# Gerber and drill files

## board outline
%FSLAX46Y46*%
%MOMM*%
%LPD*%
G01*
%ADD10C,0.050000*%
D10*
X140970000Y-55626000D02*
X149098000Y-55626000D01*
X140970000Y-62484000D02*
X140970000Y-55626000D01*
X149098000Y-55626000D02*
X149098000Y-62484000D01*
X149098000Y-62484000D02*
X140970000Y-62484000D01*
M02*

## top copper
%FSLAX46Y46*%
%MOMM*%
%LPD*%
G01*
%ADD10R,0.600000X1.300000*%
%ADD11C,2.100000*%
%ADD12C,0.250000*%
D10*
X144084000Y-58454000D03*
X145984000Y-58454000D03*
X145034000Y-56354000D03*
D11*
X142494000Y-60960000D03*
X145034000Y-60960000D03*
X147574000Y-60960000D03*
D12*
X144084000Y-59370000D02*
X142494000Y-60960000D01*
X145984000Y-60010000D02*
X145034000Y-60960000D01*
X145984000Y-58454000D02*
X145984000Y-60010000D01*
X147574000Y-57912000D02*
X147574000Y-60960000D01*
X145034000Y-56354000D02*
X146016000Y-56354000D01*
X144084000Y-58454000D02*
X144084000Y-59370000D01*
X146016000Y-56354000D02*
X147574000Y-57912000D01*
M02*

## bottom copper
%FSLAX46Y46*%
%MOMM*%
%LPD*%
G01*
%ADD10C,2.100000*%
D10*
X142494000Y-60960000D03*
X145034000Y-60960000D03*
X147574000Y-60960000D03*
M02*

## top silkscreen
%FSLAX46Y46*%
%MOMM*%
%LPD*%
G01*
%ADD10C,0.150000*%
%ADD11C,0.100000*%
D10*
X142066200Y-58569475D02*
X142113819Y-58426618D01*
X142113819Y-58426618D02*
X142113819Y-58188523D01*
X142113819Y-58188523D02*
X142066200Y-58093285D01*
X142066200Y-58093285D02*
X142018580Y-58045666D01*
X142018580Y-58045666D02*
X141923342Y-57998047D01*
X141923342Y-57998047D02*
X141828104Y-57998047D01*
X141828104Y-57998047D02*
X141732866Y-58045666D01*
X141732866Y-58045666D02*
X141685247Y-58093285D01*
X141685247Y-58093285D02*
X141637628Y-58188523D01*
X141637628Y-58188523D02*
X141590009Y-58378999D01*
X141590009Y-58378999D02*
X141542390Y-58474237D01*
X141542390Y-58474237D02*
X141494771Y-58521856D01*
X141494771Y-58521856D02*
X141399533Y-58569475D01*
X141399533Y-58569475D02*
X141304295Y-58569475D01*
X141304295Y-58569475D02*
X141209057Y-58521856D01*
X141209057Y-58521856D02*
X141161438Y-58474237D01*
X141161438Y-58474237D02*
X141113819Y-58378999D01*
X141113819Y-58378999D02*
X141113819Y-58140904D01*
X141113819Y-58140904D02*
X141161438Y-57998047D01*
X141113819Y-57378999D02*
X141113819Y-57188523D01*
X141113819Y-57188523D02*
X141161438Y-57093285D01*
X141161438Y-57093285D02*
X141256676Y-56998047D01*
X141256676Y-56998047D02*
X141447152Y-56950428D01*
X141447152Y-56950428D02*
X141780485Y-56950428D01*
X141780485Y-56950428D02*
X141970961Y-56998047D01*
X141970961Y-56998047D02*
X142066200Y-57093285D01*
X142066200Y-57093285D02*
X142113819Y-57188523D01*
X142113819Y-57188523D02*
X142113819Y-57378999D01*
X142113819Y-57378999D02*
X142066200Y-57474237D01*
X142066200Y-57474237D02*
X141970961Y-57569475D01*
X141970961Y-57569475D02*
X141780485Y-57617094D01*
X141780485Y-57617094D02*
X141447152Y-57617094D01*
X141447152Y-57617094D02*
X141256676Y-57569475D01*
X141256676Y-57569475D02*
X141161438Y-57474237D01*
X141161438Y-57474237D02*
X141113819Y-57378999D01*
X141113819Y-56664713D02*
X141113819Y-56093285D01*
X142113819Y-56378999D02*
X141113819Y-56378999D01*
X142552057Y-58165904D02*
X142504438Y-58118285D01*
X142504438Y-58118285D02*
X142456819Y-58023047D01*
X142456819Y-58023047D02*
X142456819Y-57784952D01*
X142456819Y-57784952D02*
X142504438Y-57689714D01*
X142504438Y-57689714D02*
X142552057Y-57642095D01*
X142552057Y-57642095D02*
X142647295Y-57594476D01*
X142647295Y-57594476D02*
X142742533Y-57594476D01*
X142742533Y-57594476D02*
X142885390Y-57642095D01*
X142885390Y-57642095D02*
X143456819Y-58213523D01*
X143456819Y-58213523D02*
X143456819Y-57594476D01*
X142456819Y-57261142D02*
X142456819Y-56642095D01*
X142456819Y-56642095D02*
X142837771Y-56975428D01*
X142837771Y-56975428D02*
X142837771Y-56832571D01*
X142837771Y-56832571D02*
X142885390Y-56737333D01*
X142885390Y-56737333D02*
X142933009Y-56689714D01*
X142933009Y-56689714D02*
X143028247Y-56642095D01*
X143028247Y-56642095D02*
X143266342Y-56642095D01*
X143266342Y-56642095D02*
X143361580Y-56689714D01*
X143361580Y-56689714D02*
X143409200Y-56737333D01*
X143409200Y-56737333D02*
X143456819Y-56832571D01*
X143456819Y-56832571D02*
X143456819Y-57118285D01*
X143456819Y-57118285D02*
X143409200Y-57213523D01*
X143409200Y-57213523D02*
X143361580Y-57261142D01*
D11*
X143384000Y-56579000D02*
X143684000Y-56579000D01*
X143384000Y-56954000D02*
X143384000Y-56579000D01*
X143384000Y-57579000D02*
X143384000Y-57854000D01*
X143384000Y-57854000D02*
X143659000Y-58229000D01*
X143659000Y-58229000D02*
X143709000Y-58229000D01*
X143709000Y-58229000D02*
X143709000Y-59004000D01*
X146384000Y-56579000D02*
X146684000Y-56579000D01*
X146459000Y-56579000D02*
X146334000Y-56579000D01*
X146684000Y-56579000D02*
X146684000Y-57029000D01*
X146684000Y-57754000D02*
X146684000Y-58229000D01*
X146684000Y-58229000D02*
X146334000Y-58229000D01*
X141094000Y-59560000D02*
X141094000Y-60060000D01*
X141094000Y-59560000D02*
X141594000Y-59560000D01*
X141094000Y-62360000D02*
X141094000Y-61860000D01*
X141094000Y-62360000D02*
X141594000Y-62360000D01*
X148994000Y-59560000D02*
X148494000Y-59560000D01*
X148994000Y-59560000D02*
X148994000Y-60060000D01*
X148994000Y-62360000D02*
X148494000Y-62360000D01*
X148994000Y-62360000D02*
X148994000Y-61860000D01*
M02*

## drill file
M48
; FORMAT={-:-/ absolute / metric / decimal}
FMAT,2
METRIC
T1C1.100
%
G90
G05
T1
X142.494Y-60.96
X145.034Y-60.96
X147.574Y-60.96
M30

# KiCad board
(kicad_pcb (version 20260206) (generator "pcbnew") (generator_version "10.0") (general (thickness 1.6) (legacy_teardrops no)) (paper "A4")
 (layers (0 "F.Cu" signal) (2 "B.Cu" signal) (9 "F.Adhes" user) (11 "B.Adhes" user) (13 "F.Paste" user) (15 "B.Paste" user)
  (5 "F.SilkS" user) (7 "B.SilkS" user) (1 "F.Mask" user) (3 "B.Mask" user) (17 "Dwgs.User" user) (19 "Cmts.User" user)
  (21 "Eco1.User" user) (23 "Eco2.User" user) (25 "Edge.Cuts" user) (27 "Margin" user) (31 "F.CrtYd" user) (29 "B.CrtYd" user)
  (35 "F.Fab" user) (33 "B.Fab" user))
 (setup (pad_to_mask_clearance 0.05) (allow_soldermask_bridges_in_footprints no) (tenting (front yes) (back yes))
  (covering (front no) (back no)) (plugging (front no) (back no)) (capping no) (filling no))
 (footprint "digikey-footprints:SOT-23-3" (layer "F.Cu") (at 145.034 57.404 90)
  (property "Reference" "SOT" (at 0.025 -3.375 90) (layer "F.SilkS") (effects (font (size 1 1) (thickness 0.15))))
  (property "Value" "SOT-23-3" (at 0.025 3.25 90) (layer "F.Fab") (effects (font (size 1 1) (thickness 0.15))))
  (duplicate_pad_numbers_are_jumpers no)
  (fp_line (start 0.825 -1.65) (end 0.825 -1.35) (stroke (width 0.1) (type solid)) (layer "F.SilkS"))
  (fp_line (start 0.45 -1.65) (end 0.825 -1.65) (stroke (width 0.1) (type solid)) (layer "F.SilkS"))
  (fp_line (start -0.175 -1.65) (end -0.45 -1.65) (stroke (width 0.1) (type solid)) (layer "F.SilkS"))
  (fp_line (start -0.45 -1.65) (end -0.825 -1.375) (stroke (width 0.1) (type solid)) (layer "F.SilkS"))
  (fp_line (start -0.825 -1.375) (end -0.825 -1.325) (stroke (width 0.1) (type solid)) (layer "F.SilkS"))
  (fp_line (start -0.825 -1.325) (end -1.6 -1.325) (stroke (width 0.1) (type solid)) (layer "F.SilkS"))
  (fp_line (start 0.825 1.35) (end 0.825 1.65) (stroke (width 0.1) (type solid)) (layer "F.SilkS"))
  (fp_line (start 0.825 1.425) (end 0.825 1.3) (stroke (width 0.1) (type solid)) (layer "F.SilkS"))
  (fp_line (start 0.825 1.65) (end 0.375 1.65) (stroke (width 0.1) (type solid)) (layer "F.SilkS"))
  (fp_line (start -0.35 1.65) (end -0.825 1.65) (stroke (width 0.1) (type solid)) (layer "F.SilkS"))
  (fp_line (start -0.825 1.65) (end -0.825 1.3) (stroke (width 0.1) (type solid)) (layer "F.SilkS"))
  (pad "1" smd rect (at -1.05 -0.95 90) (size 1.3 0.6) (layers "F.Cu" "F.Mask" "F.Paste") (solder_mask_margin 0.07))
  (pad "2" smd rect (at -1.05 0.95 90) (size 1.3 0.6) (layers "F.Cu" "F.Mask" "F.Paste") (solder_mask_margin 0.07))
  (pad "3" smd rect (at 1.05 0 90) (size 1.3 0.6) (layers "F.Cu" "F.Mask" "F.Paste") (solder_mask_margin 0.07)))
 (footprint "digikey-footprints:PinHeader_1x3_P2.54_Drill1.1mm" (layer "F.Cu") (at 142.494 60.96)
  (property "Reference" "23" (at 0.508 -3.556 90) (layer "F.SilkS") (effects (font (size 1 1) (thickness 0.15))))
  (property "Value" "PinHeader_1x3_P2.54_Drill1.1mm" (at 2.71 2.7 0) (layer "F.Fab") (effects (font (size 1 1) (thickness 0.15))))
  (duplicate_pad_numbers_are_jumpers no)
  (fp_line (start -1.4 -1.4) (end -1.4 -0.9) (stroke (width 0.1) (type solid)) (layer "F.SilkS"))
  (fp_line (start -1.4 -1.4) (end -0.9 -1.4) (stroke (width 0.1) (type solid)) (layer "F.SilkS"))
  (fp_line (start -1.4 1.4) (end -1.4 0.9) (stroke (width 0.1) (type solid)) (layer "F.SilkS"))
  (fp_line (start -1.4 1.4) (end -0.9 1.4) (stroke (width 0.1) (type solid)) (layer "F.SilkS"))
  (fp_line (start 6.5 -1.4) (end 6 -1.4) (stroke (width 0.1) (type solid)) (layer "F.SilkS"))
  (fp_line (start 6.5 -1.4) (end 6.5 -0.9) (stroke (width 0.1) (type solid)) (layer "F.SilkS"))
  (fp_line (start 6.5 1.4) (end 6 1.4) (stroke (width 0.1) (type solid)) (layer "F.SilkS"))
  (fp_line (start 6.5 1.4) (end 6.5 0.9) (stroke (width 0.1) (type solid)) (layer "F.SilkS"))
  (pad "1" thru_hole circle (at 0 0) (size 2.1 2.1) (drill 1.1) (layers "*.Cu" "*.Mask") (remove_unused_layers no))
  (pad "2" thru_hole circle (at 2.54 0) (size 2.1 2.1) (drill 1.1) (layers "*.Cu" "*.Mask") (remove_unused_layers no))
  (pad "3" thru_hole circle (at 5.08 0) (size 2.1 2.1) (drill 1.1) (layers "*.Cu" "*.Mask") (remove_unused_layers no)))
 (gr_line (start 140.97 55.626) (end 149.098 55.626) (stroke (width 0.05) (type solid)) (layer "Edge.Cuts"))
 (gr_line (start 140.97 62.484) (end 140.97 55.626) (stroke (width 0.05) (type solid)) (layer "Edge.Cuts"))
 (gr_line (start 149.098 55.626) (end 149.098 62.484) (stroke (width 0.05) (type solid)) (layer "Edge.Cuts"))
 (gr_line (start 149.098 62.484) (end 140.97 62.484) (stroke (width 0.05) (type solid)) (layer "Edge.Cuts"))
 (segment (start 144.084 59.37) (end 142.494 60.96) (width 0.25) (layer "F.Cu") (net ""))
 (segment (start 145.984 60.01) (end 145.034 60.96) (width 0.25) (layer "F.Cu") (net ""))
 (segment (start 145.984 58.454) (end 145.984 60.01) (width 0.25) (layer "F.Cu") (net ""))
 (segment (start 147.574 57.912) (end 147.574 60.96) (width 0.25) (layer "F.Cu") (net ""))
 (segment (start 145.034 56.354) (end 146.016 56.354) (width 0.25) (layer "F.Cu") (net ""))
 (segment (start 144.084 58.454) (end 144.084 59.37) (width 0.25) (layer "F.Cu") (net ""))
 (segment (start 146.016 56.354) (end 147.574 57.912) (width 0.25) (layer "F.Cu") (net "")))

